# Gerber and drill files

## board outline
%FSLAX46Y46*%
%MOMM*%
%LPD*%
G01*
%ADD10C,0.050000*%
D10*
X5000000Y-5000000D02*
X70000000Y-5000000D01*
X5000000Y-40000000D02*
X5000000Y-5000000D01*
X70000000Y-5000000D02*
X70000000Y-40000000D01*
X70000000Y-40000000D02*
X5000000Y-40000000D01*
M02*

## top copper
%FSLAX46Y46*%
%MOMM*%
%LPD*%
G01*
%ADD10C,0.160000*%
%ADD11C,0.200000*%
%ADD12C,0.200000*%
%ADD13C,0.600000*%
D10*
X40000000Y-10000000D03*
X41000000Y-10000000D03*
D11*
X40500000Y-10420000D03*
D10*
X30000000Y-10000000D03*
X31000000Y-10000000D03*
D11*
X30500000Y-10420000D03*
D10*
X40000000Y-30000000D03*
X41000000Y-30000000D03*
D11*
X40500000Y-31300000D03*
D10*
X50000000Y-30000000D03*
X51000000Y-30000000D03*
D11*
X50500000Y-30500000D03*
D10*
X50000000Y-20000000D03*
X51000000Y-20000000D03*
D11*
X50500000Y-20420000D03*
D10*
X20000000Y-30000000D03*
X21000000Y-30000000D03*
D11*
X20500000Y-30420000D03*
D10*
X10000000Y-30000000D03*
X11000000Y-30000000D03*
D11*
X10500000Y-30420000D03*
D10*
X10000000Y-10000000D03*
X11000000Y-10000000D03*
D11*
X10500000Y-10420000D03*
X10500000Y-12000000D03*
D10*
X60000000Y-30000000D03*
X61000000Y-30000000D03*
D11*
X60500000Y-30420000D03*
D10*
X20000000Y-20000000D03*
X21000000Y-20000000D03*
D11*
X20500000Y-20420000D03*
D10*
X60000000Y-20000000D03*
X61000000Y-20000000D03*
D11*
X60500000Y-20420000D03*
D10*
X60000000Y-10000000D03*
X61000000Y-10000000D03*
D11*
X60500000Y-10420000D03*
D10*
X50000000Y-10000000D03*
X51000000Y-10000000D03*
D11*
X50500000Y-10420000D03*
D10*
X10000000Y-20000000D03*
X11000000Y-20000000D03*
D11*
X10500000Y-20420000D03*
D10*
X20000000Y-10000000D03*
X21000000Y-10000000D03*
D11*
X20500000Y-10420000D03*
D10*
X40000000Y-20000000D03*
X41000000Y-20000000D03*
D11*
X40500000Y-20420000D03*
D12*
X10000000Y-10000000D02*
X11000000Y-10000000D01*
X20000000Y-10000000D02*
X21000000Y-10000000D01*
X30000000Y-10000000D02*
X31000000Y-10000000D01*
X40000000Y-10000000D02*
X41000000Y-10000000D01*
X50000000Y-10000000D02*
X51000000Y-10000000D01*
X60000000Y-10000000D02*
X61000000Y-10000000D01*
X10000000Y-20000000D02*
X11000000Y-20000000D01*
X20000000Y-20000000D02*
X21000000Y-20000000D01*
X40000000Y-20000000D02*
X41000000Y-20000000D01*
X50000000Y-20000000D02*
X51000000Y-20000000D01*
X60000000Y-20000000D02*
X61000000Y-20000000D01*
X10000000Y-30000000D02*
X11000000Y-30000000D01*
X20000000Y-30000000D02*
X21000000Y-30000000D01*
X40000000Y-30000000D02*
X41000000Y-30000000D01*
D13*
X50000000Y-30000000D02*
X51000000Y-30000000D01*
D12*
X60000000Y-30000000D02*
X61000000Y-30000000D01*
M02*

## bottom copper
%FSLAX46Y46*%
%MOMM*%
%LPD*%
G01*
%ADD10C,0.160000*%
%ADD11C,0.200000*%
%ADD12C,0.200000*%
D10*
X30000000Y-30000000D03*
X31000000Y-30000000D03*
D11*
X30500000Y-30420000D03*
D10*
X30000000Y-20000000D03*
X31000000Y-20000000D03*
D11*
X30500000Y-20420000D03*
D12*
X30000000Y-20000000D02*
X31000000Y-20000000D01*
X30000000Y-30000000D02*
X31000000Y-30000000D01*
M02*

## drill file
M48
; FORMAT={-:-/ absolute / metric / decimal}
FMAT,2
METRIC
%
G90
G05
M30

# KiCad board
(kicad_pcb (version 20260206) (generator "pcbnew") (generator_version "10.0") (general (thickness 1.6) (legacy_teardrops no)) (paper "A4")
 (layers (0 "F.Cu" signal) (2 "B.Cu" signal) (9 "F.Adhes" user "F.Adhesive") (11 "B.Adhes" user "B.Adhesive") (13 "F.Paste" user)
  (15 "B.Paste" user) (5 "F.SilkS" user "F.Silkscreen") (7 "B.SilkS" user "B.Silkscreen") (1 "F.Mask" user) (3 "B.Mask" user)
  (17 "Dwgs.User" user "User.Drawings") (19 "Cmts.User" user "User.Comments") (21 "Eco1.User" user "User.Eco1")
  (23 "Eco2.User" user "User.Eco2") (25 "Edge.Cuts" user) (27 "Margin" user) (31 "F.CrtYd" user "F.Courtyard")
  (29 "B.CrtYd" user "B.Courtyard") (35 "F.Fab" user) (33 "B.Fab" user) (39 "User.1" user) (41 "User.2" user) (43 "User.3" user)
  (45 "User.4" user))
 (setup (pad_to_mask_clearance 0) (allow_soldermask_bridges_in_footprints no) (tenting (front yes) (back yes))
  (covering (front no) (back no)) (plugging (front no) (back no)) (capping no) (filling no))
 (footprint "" (layer "F.Cu") (at 30 30)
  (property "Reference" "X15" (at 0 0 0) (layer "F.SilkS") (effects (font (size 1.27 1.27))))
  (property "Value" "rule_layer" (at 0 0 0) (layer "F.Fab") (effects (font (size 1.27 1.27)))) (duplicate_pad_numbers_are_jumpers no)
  (pad "1" smd circle (at 0 0) (size 0.16 0.16) (layers "B.Cu") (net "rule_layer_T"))
  (pad "2" smd circle (at 1 0) (size 0.16 0.16) (layers "B.Cu") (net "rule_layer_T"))
  (pad "3" smd circle (at 0.5 0.42) (size 0.2 0.2) (layers "B.Cu") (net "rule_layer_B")))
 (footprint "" (layer "F.Cu") (at 40 10)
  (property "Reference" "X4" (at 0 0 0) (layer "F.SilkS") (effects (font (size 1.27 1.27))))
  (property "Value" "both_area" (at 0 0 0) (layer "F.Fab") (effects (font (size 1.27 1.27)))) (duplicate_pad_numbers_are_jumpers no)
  (pad "1" smd circle (at 0 0) (size 0.16 0.16) (layers "F.Cu") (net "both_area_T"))
  (pad "2" smd circle (at 1 0) (size 0.16 0.16) (layers "F.Cu") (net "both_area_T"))
  (pad "3" smd circle (at 0.5 0.42) (size 0.2 0.2) (layers "F.Cu") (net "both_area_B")))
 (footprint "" (layer "F.Cu") (at 30 10)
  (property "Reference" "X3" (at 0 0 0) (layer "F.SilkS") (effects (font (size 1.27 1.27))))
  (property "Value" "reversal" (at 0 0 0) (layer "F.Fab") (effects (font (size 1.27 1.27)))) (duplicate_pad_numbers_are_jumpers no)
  (pad "1" smd circle (at 0 0) (size 0.16 0.16) (layers "F.Cu") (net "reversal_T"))
  (pad "2" smd circle (at 1 0) (size 0.16 0.16) (layers "F.Cu") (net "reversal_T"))
  (pad "3" smd circle (at 0.5 0.42) (size 0.2 0.2) (layers "F.Cu") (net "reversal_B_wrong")))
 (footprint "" (layer "F.Cu") (at 40 30)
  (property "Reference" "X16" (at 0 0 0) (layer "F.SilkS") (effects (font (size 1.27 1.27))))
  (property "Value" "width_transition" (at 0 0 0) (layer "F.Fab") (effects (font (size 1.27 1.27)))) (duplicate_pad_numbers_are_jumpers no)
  (pad "1" smd circle (at 0 0) (size 0.16 0.16) (layers "F.Cu") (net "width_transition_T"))
  (pad "2" smd circle (at 1 0) (size 0.16 0.16) (layers "F.Cu") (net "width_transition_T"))
  (pad "3" smd circle (at 0.5 1.3) (size 0.2 0.2) (layers "F.Cu") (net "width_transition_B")))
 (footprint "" (layer "F.Cu") (at 50 30)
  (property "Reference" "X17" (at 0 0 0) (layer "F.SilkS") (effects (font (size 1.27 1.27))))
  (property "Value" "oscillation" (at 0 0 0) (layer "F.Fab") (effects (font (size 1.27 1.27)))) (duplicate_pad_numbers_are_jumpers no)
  (pad "1" smd circle (at 0 0) (size 0.16 0.16) (layers "F.Cu") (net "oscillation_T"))
  (pad "2" smd circle (at 1 0) (size 0.16 0.16) (layers "F.Cu") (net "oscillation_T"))
  (pad "3" smd circle (at 0.5 0.5) (size 0.2 0.2) (layers "F.Cu") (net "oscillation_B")))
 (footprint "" (layer "F.Cu") (at 50 20)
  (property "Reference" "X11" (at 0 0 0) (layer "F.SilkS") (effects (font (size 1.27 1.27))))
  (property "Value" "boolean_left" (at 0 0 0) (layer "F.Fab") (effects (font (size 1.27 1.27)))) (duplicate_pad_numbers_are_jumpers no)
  (pad "1" smd circle (at 0 0) (size 0.16 0.16) (layers "F.Cu") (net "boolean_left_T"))
  (pad "2" smd circle (at 1 0) (size 0.16 0.16) (layers "F.Cu") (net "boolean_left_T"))
  (pad "3" smd circle (at 0.5 0.42) (size 0.2 0.2) (layers "F.Cu") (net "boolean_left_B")))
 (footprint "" (layer "F.Cu") (at 20 30)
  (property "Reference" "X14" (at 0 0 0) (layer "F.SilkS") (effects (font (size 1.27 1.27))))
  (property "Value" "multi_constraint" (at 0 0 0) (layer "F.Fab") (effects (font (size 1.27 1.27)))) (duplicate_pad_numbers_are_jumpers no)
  (pad "1" smd circle (at 0 0) (size 0.16 0.16) (layers "F.Cu") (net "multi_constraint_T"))
  (pad "2" smd circle (at 1 0) (size 0.16 0.16) (layers "F.Cu") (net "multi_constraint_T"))
  (pad "3" smd circle (at 0.5 0.42) (size 0.2 0.2) (layers "F.Cu") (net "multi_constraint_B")))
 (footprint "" (layer "F.Cu") (at 10 30)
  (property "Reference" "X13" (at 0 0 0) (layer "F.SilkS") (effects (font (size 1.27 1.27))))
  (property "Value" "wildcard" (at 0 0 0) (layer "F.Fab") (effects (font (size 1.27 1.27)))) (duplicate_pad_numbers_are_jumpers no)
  (pad "1" smd circle (at 0 0) (size 0.16 0.16) (layers "F.Cu") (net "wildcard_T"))
  (pad "2" smd circle (at 1 0) (size 0.16 0.16) (layers "F.Cu") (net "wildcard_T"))
  (pad "3" smd circle (at 0.5 0.42) (size 0.2 0.2) (layers "F.Cu") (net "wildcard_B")))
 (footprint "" (layer "F.Cu") (at 10 10)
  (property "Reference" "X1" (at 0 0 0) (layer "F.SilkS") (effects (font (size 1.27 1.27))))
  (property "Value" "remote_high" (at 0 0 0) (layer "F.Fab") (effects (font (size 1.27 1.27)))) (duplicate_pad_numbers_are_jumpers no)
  (pad "1" smd circle (at 0 0) (size 0.16 0.16) (layers "F.Cu") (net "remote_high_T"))
  (pad "2" smd circle (at 1 0) (size 0.16 0.16) (layers "F.Cu") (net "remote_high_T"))
  (pad "3" smd circle (at 0.5 0.42) (size 0.2 0.2) (layers "F.Cu") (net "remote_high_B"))
  (pad "4" smd circle (at 0.5 2) (size 0.2 0.2) (layers "F.Cu") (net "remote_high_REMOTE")))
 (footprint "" (layer "F.Cu") (at 60 30)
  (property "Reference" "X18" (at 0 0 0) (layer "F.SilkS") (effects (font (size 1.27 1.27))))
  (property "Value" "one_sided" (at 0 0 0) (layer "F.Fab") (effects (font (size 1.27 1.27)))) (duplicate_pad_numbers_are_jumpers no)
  (pad "1" smd circle (at 0 0) (size 0.16 0.16) (layers "F.Cu") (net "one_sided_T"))
  (pad "2" smd circle (at 1 0) (size 0.16 0.16) (layers "F.Cu") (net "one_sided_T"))
  (pad "3" smd circle (at 0.5 0.42) (size 0.2 0.2) (layers "F.Cu") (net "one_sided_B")))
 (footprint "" (layer "F.Cu") (at 20 20)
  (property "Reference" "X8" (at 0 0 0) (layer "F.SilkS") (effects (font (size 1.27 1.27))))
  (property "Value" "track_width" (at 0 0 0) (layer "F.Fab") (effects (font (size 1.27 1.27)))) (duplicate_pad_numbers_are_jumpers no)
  (pad "1" smd circle (at 0 0) (size 0.16 0.16) (layers "F.Cu") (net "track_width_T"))
  (pad "2" smd circle (at 1 0) (size 0.16 0.16) (layers "F.Cu") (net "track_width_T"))
  (pad "3" smd circle (at 0.5 0.42) (size 0.2 0.2) (layers "F.Cu") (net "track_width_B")))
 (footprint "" (layer "F.Cu") (at 60 20)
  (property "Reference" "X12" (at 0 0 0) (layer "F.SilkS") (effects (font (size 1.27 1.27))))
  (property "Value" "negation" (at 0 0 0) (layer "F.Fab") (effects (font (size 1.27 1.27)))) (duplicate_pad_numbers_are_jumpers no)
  (pad "1" smd circle (at 0 0) (size 0.16 0.16) (layers "F.Cu") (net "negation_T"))
  (pad "2" smd circle (at 1 0) (size 0.16 0.16) (layers "F.Cu") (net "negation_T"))
  (pad "3" smd circle (at 0.5 0.42) (size 0.2 0.2) (layers "F.Cu") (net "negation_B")))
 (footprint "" (layer "F.Cu") (at 60 10)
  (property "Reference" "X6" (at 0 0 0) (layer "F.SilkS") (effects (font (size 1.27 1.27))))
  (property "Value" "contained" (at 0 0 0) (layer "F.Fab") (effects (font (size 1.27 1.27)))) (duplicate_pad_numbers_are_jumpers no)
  (pad "1" smd circle (at 0 0) (size 0.16 0.16) (layers "F.Cu") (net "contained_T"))
  (pad "2" smd circle (at 1 0) (size 0.16 0.16) (layers "F.Cu") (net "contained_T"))
  (pad "3" smd circle (at 0.5 0.42) (size 0.2 0.2) (layers "F.Cu") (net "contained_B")))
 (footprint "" (layer "F.Cu") (at 50 10)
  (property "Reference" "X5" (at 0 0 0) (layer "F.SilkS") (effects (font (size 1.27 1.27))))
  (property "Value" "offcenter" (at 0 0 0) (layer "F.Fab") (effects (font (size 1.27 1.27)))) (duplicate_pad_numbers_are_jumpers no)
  (pad "1" smd circle (at 0 0) (size 0.16 0.16) (layers "F.Cu") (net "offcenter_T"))
  (pad "2" smd circle (at 1 0) (size 0.16 0.16) (layers "F.Cu") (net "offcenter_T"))
  (pad "3" smd circle (at 0.5 0.42) (size 0.2 0.2) (layers "F.Cu") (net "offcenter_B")))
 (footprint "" (layer "F.Cu") (at 10 20)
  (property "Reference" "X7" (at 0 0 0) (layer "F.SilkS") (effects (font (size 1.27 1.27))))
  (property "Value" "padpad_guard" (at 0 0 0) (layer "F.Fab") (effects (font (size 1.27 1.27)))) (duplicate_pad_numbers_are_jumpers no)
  (pad "1" smd circle (at 0 0) (size 0.16 0.16) (layers "F.Cu") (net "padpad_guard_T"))
  (pad "2" smd circle (at 1 0) (size 0.16 0.16) (layers "F.Cu") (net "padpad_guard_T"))
  (pad "3" smd circle (at 0.5 0.42) (size 0.2 0.2) (layers "F.Cu") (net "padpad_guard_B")))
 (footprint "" (layer "F.Cu") (at 20 10)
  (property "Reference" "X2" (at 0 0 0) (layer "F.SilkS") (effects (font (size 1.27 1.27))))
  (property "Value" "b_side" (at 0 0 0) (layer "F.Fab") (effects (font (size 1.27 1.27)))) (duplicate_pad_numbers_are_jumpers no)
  (pad "1" smd circle (at 0 0) (size 0.16 0.16) (layers "F.Cu") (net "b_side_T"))
  (pad "2" smd circle (at 1 0) (size 0.16 0.16) (layers "F.Cu") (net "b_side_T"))
  (pad "3" smd circle (at 0.5 0.42) (size 0.2 0.2) (layers "F.Cu") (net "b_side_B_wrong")))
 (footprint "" (layer "F.Cu") (at 40 20)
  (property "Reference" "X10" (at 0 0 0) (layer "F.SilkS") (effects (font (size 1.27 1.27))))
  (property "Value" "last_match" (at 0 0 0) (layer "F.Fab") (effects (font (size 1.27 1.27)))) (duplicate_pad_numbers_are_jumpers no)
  (pad "1" smd circle (at 0 0) (size 0.16 0.16) (layers "F.Cu") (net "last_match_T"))
  (pad "2" smd circle (at 1 0) (size 0.16 0.16) (layers "F.Cu") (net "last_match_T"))
  (pad "3" smd circle (at 0.5 0.42) (size 0.2 0.2) (layers "F.Cu") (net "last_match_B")))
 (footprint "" (layer "F.Cu") (at 30 20)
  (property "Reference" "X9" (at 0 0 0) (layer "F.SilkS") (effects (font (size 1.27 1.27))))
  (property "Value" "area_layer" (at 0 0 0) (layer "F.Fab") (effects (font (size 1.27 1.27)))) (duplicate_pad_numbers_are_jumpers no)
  (pad "1" smd circle (at 0 0) (size 0.16 0.16) (layers "B.Cu") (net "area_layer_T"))
  (pad "2" smd circle (at 1 0) (size 0.16 0.16) (layers "B.Cu") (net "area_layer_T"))
  (pad "3" smd circle (at 0.5 0.42) (size 0.2 0.2) (layers "B.Cu") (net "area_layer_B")))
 (gr_line (start 5 5) (end 70 5) (stroke (width 0.05) (type default)) (layer "Edge.Cuts"))
 (gr_line (start 5 40) (end 5 5) (stroke (width 0.05) (type default)) (layer "Edge.Cuts"))
 (gr_line (start 70 5) (end 70 40) (stroke (width 0.05) (type default)) (layer "Edge.Cuts"))
 (gr_line (start 70 40) (end 5 40) (stroke (width 0.05) (type default)) (layer "Edge.Cuts"))
 (segment (start 10 10) (end 11 10) (width 0.2) (layer "F.Cu") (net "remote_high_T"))
 (segment (start 20 10) (end 21 10) (width 0.2) (layer "F.Cu") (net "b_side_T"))
 (segment (start 30 10) (end 31 10) (width 0.2) (layer "F.Cu") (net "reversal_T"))
 (segment (start 40 10) (end 41 10) (width 0.2) (layer "F.Cu") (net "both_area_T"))
 (segment (start 50 10) (end 51 10) (width 0.2) (layer "F.Cu") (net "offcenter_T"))
 (segment (start 60 10) (end 61 10) (width 0.2) (layer "F.Cu") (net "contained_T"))
 (segment (start 10 20) (end 11 20) (width 0.2) (layer "F.Cu") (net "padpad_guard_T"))
 (segment (start 20 20) (end 21 20) (width 0.2) (layer "F.Cu") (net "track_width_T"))
 (segment (start 30 20) (end 31 20) (width 0.2) (layer "B.Cu") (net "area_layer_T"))
 (segment (start 40 20) (end 41 20) (width 0.2) (layer "F.Cu") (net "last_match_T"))
 (segment (start 50 20) (end 51 20) (width 0.2) (layer "F.Cu") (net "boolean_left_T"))
 (segment (start 60 20) (end 61 20) (width 0.2) (layer "F.Cu") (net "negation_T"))
 (segment (start 10 30) (end 11 30) (width 0.2) (layer "F.Cu") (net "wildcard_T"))
 (segment (start 20 30) (end 21 30) (width 0.2) (layer "F.Cu") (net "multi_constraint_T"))
 (segment (start 30 30) (end 31 30) (width 0.2) (layer "B.Cu") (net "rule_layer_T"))
 (segment (start 40 30) (end 41 30) (width 0.2) (layer "F.Cu") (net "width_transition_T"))
 (segment (start 50 30) (end 51 30) (width 0.6) (layer "F.Cu") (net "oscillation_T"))
 (segment (start 60 30) (end 61 30) (width 0.2) (layer "F.Cu") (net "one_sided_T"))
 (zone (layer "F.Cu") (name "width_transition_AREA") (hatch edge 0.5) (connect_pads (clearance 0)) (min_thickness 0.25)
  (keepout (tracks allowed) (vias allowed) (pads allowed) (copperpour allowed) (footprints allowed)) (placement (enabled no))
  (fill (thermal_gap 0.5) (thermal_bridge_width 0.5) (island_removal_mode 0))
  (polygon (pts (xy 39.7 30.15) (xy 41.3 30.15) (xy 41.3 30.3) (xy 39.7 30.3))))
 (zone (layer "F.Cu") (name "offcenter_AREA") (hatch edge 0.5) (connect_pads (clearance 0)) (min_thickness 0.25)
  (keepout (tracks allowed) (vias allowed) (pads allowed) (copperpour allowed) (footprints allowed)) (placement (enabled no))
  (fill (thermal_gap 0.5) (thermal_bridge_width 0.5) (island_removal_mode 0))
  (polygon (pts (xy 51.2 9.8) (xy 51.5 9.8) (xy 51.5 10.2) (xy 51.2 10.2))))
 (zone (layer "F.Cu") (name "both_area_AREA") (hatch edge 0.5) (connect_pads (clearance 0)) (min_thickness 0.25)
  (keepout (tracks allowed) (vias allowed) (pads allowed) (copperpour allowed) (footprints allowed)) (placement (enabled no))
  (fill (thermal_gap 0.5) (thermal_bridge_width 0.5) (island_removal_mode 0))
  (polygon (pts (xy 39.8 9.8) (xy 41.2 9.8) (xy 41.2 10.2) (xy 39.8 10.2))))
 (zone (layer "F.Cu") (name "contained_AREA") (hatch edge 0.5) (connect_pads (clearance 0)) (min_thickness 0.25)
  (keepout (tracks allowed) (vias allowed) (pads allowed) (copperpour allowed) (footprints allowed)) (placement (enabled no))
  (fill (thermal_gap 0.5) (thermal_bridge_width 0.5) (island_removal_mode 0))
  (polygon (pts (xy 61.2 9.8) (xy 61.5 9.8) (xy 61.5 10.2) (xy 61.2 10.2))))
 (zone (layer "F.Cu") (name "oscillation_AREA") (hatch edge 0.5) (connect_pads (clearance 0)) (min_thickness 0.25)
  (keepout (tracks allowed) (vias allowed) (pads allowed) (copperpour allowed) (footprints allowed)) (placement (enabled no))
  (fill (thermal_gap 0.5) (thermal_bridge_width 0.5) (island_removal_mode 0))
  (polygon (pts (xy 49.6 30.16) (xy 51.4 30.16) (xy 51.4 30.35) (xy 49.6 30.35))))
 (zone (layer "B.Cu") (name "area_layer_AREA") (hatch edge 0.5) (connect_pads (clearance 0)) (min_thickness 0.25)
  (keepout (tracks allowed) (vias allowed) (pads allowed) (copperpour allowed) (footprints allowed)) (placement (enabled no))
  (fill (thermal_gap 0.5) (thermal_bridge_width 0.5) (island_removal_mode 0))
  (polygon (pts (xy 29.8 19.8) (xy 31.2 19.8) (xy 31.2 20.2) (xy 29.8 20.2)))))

